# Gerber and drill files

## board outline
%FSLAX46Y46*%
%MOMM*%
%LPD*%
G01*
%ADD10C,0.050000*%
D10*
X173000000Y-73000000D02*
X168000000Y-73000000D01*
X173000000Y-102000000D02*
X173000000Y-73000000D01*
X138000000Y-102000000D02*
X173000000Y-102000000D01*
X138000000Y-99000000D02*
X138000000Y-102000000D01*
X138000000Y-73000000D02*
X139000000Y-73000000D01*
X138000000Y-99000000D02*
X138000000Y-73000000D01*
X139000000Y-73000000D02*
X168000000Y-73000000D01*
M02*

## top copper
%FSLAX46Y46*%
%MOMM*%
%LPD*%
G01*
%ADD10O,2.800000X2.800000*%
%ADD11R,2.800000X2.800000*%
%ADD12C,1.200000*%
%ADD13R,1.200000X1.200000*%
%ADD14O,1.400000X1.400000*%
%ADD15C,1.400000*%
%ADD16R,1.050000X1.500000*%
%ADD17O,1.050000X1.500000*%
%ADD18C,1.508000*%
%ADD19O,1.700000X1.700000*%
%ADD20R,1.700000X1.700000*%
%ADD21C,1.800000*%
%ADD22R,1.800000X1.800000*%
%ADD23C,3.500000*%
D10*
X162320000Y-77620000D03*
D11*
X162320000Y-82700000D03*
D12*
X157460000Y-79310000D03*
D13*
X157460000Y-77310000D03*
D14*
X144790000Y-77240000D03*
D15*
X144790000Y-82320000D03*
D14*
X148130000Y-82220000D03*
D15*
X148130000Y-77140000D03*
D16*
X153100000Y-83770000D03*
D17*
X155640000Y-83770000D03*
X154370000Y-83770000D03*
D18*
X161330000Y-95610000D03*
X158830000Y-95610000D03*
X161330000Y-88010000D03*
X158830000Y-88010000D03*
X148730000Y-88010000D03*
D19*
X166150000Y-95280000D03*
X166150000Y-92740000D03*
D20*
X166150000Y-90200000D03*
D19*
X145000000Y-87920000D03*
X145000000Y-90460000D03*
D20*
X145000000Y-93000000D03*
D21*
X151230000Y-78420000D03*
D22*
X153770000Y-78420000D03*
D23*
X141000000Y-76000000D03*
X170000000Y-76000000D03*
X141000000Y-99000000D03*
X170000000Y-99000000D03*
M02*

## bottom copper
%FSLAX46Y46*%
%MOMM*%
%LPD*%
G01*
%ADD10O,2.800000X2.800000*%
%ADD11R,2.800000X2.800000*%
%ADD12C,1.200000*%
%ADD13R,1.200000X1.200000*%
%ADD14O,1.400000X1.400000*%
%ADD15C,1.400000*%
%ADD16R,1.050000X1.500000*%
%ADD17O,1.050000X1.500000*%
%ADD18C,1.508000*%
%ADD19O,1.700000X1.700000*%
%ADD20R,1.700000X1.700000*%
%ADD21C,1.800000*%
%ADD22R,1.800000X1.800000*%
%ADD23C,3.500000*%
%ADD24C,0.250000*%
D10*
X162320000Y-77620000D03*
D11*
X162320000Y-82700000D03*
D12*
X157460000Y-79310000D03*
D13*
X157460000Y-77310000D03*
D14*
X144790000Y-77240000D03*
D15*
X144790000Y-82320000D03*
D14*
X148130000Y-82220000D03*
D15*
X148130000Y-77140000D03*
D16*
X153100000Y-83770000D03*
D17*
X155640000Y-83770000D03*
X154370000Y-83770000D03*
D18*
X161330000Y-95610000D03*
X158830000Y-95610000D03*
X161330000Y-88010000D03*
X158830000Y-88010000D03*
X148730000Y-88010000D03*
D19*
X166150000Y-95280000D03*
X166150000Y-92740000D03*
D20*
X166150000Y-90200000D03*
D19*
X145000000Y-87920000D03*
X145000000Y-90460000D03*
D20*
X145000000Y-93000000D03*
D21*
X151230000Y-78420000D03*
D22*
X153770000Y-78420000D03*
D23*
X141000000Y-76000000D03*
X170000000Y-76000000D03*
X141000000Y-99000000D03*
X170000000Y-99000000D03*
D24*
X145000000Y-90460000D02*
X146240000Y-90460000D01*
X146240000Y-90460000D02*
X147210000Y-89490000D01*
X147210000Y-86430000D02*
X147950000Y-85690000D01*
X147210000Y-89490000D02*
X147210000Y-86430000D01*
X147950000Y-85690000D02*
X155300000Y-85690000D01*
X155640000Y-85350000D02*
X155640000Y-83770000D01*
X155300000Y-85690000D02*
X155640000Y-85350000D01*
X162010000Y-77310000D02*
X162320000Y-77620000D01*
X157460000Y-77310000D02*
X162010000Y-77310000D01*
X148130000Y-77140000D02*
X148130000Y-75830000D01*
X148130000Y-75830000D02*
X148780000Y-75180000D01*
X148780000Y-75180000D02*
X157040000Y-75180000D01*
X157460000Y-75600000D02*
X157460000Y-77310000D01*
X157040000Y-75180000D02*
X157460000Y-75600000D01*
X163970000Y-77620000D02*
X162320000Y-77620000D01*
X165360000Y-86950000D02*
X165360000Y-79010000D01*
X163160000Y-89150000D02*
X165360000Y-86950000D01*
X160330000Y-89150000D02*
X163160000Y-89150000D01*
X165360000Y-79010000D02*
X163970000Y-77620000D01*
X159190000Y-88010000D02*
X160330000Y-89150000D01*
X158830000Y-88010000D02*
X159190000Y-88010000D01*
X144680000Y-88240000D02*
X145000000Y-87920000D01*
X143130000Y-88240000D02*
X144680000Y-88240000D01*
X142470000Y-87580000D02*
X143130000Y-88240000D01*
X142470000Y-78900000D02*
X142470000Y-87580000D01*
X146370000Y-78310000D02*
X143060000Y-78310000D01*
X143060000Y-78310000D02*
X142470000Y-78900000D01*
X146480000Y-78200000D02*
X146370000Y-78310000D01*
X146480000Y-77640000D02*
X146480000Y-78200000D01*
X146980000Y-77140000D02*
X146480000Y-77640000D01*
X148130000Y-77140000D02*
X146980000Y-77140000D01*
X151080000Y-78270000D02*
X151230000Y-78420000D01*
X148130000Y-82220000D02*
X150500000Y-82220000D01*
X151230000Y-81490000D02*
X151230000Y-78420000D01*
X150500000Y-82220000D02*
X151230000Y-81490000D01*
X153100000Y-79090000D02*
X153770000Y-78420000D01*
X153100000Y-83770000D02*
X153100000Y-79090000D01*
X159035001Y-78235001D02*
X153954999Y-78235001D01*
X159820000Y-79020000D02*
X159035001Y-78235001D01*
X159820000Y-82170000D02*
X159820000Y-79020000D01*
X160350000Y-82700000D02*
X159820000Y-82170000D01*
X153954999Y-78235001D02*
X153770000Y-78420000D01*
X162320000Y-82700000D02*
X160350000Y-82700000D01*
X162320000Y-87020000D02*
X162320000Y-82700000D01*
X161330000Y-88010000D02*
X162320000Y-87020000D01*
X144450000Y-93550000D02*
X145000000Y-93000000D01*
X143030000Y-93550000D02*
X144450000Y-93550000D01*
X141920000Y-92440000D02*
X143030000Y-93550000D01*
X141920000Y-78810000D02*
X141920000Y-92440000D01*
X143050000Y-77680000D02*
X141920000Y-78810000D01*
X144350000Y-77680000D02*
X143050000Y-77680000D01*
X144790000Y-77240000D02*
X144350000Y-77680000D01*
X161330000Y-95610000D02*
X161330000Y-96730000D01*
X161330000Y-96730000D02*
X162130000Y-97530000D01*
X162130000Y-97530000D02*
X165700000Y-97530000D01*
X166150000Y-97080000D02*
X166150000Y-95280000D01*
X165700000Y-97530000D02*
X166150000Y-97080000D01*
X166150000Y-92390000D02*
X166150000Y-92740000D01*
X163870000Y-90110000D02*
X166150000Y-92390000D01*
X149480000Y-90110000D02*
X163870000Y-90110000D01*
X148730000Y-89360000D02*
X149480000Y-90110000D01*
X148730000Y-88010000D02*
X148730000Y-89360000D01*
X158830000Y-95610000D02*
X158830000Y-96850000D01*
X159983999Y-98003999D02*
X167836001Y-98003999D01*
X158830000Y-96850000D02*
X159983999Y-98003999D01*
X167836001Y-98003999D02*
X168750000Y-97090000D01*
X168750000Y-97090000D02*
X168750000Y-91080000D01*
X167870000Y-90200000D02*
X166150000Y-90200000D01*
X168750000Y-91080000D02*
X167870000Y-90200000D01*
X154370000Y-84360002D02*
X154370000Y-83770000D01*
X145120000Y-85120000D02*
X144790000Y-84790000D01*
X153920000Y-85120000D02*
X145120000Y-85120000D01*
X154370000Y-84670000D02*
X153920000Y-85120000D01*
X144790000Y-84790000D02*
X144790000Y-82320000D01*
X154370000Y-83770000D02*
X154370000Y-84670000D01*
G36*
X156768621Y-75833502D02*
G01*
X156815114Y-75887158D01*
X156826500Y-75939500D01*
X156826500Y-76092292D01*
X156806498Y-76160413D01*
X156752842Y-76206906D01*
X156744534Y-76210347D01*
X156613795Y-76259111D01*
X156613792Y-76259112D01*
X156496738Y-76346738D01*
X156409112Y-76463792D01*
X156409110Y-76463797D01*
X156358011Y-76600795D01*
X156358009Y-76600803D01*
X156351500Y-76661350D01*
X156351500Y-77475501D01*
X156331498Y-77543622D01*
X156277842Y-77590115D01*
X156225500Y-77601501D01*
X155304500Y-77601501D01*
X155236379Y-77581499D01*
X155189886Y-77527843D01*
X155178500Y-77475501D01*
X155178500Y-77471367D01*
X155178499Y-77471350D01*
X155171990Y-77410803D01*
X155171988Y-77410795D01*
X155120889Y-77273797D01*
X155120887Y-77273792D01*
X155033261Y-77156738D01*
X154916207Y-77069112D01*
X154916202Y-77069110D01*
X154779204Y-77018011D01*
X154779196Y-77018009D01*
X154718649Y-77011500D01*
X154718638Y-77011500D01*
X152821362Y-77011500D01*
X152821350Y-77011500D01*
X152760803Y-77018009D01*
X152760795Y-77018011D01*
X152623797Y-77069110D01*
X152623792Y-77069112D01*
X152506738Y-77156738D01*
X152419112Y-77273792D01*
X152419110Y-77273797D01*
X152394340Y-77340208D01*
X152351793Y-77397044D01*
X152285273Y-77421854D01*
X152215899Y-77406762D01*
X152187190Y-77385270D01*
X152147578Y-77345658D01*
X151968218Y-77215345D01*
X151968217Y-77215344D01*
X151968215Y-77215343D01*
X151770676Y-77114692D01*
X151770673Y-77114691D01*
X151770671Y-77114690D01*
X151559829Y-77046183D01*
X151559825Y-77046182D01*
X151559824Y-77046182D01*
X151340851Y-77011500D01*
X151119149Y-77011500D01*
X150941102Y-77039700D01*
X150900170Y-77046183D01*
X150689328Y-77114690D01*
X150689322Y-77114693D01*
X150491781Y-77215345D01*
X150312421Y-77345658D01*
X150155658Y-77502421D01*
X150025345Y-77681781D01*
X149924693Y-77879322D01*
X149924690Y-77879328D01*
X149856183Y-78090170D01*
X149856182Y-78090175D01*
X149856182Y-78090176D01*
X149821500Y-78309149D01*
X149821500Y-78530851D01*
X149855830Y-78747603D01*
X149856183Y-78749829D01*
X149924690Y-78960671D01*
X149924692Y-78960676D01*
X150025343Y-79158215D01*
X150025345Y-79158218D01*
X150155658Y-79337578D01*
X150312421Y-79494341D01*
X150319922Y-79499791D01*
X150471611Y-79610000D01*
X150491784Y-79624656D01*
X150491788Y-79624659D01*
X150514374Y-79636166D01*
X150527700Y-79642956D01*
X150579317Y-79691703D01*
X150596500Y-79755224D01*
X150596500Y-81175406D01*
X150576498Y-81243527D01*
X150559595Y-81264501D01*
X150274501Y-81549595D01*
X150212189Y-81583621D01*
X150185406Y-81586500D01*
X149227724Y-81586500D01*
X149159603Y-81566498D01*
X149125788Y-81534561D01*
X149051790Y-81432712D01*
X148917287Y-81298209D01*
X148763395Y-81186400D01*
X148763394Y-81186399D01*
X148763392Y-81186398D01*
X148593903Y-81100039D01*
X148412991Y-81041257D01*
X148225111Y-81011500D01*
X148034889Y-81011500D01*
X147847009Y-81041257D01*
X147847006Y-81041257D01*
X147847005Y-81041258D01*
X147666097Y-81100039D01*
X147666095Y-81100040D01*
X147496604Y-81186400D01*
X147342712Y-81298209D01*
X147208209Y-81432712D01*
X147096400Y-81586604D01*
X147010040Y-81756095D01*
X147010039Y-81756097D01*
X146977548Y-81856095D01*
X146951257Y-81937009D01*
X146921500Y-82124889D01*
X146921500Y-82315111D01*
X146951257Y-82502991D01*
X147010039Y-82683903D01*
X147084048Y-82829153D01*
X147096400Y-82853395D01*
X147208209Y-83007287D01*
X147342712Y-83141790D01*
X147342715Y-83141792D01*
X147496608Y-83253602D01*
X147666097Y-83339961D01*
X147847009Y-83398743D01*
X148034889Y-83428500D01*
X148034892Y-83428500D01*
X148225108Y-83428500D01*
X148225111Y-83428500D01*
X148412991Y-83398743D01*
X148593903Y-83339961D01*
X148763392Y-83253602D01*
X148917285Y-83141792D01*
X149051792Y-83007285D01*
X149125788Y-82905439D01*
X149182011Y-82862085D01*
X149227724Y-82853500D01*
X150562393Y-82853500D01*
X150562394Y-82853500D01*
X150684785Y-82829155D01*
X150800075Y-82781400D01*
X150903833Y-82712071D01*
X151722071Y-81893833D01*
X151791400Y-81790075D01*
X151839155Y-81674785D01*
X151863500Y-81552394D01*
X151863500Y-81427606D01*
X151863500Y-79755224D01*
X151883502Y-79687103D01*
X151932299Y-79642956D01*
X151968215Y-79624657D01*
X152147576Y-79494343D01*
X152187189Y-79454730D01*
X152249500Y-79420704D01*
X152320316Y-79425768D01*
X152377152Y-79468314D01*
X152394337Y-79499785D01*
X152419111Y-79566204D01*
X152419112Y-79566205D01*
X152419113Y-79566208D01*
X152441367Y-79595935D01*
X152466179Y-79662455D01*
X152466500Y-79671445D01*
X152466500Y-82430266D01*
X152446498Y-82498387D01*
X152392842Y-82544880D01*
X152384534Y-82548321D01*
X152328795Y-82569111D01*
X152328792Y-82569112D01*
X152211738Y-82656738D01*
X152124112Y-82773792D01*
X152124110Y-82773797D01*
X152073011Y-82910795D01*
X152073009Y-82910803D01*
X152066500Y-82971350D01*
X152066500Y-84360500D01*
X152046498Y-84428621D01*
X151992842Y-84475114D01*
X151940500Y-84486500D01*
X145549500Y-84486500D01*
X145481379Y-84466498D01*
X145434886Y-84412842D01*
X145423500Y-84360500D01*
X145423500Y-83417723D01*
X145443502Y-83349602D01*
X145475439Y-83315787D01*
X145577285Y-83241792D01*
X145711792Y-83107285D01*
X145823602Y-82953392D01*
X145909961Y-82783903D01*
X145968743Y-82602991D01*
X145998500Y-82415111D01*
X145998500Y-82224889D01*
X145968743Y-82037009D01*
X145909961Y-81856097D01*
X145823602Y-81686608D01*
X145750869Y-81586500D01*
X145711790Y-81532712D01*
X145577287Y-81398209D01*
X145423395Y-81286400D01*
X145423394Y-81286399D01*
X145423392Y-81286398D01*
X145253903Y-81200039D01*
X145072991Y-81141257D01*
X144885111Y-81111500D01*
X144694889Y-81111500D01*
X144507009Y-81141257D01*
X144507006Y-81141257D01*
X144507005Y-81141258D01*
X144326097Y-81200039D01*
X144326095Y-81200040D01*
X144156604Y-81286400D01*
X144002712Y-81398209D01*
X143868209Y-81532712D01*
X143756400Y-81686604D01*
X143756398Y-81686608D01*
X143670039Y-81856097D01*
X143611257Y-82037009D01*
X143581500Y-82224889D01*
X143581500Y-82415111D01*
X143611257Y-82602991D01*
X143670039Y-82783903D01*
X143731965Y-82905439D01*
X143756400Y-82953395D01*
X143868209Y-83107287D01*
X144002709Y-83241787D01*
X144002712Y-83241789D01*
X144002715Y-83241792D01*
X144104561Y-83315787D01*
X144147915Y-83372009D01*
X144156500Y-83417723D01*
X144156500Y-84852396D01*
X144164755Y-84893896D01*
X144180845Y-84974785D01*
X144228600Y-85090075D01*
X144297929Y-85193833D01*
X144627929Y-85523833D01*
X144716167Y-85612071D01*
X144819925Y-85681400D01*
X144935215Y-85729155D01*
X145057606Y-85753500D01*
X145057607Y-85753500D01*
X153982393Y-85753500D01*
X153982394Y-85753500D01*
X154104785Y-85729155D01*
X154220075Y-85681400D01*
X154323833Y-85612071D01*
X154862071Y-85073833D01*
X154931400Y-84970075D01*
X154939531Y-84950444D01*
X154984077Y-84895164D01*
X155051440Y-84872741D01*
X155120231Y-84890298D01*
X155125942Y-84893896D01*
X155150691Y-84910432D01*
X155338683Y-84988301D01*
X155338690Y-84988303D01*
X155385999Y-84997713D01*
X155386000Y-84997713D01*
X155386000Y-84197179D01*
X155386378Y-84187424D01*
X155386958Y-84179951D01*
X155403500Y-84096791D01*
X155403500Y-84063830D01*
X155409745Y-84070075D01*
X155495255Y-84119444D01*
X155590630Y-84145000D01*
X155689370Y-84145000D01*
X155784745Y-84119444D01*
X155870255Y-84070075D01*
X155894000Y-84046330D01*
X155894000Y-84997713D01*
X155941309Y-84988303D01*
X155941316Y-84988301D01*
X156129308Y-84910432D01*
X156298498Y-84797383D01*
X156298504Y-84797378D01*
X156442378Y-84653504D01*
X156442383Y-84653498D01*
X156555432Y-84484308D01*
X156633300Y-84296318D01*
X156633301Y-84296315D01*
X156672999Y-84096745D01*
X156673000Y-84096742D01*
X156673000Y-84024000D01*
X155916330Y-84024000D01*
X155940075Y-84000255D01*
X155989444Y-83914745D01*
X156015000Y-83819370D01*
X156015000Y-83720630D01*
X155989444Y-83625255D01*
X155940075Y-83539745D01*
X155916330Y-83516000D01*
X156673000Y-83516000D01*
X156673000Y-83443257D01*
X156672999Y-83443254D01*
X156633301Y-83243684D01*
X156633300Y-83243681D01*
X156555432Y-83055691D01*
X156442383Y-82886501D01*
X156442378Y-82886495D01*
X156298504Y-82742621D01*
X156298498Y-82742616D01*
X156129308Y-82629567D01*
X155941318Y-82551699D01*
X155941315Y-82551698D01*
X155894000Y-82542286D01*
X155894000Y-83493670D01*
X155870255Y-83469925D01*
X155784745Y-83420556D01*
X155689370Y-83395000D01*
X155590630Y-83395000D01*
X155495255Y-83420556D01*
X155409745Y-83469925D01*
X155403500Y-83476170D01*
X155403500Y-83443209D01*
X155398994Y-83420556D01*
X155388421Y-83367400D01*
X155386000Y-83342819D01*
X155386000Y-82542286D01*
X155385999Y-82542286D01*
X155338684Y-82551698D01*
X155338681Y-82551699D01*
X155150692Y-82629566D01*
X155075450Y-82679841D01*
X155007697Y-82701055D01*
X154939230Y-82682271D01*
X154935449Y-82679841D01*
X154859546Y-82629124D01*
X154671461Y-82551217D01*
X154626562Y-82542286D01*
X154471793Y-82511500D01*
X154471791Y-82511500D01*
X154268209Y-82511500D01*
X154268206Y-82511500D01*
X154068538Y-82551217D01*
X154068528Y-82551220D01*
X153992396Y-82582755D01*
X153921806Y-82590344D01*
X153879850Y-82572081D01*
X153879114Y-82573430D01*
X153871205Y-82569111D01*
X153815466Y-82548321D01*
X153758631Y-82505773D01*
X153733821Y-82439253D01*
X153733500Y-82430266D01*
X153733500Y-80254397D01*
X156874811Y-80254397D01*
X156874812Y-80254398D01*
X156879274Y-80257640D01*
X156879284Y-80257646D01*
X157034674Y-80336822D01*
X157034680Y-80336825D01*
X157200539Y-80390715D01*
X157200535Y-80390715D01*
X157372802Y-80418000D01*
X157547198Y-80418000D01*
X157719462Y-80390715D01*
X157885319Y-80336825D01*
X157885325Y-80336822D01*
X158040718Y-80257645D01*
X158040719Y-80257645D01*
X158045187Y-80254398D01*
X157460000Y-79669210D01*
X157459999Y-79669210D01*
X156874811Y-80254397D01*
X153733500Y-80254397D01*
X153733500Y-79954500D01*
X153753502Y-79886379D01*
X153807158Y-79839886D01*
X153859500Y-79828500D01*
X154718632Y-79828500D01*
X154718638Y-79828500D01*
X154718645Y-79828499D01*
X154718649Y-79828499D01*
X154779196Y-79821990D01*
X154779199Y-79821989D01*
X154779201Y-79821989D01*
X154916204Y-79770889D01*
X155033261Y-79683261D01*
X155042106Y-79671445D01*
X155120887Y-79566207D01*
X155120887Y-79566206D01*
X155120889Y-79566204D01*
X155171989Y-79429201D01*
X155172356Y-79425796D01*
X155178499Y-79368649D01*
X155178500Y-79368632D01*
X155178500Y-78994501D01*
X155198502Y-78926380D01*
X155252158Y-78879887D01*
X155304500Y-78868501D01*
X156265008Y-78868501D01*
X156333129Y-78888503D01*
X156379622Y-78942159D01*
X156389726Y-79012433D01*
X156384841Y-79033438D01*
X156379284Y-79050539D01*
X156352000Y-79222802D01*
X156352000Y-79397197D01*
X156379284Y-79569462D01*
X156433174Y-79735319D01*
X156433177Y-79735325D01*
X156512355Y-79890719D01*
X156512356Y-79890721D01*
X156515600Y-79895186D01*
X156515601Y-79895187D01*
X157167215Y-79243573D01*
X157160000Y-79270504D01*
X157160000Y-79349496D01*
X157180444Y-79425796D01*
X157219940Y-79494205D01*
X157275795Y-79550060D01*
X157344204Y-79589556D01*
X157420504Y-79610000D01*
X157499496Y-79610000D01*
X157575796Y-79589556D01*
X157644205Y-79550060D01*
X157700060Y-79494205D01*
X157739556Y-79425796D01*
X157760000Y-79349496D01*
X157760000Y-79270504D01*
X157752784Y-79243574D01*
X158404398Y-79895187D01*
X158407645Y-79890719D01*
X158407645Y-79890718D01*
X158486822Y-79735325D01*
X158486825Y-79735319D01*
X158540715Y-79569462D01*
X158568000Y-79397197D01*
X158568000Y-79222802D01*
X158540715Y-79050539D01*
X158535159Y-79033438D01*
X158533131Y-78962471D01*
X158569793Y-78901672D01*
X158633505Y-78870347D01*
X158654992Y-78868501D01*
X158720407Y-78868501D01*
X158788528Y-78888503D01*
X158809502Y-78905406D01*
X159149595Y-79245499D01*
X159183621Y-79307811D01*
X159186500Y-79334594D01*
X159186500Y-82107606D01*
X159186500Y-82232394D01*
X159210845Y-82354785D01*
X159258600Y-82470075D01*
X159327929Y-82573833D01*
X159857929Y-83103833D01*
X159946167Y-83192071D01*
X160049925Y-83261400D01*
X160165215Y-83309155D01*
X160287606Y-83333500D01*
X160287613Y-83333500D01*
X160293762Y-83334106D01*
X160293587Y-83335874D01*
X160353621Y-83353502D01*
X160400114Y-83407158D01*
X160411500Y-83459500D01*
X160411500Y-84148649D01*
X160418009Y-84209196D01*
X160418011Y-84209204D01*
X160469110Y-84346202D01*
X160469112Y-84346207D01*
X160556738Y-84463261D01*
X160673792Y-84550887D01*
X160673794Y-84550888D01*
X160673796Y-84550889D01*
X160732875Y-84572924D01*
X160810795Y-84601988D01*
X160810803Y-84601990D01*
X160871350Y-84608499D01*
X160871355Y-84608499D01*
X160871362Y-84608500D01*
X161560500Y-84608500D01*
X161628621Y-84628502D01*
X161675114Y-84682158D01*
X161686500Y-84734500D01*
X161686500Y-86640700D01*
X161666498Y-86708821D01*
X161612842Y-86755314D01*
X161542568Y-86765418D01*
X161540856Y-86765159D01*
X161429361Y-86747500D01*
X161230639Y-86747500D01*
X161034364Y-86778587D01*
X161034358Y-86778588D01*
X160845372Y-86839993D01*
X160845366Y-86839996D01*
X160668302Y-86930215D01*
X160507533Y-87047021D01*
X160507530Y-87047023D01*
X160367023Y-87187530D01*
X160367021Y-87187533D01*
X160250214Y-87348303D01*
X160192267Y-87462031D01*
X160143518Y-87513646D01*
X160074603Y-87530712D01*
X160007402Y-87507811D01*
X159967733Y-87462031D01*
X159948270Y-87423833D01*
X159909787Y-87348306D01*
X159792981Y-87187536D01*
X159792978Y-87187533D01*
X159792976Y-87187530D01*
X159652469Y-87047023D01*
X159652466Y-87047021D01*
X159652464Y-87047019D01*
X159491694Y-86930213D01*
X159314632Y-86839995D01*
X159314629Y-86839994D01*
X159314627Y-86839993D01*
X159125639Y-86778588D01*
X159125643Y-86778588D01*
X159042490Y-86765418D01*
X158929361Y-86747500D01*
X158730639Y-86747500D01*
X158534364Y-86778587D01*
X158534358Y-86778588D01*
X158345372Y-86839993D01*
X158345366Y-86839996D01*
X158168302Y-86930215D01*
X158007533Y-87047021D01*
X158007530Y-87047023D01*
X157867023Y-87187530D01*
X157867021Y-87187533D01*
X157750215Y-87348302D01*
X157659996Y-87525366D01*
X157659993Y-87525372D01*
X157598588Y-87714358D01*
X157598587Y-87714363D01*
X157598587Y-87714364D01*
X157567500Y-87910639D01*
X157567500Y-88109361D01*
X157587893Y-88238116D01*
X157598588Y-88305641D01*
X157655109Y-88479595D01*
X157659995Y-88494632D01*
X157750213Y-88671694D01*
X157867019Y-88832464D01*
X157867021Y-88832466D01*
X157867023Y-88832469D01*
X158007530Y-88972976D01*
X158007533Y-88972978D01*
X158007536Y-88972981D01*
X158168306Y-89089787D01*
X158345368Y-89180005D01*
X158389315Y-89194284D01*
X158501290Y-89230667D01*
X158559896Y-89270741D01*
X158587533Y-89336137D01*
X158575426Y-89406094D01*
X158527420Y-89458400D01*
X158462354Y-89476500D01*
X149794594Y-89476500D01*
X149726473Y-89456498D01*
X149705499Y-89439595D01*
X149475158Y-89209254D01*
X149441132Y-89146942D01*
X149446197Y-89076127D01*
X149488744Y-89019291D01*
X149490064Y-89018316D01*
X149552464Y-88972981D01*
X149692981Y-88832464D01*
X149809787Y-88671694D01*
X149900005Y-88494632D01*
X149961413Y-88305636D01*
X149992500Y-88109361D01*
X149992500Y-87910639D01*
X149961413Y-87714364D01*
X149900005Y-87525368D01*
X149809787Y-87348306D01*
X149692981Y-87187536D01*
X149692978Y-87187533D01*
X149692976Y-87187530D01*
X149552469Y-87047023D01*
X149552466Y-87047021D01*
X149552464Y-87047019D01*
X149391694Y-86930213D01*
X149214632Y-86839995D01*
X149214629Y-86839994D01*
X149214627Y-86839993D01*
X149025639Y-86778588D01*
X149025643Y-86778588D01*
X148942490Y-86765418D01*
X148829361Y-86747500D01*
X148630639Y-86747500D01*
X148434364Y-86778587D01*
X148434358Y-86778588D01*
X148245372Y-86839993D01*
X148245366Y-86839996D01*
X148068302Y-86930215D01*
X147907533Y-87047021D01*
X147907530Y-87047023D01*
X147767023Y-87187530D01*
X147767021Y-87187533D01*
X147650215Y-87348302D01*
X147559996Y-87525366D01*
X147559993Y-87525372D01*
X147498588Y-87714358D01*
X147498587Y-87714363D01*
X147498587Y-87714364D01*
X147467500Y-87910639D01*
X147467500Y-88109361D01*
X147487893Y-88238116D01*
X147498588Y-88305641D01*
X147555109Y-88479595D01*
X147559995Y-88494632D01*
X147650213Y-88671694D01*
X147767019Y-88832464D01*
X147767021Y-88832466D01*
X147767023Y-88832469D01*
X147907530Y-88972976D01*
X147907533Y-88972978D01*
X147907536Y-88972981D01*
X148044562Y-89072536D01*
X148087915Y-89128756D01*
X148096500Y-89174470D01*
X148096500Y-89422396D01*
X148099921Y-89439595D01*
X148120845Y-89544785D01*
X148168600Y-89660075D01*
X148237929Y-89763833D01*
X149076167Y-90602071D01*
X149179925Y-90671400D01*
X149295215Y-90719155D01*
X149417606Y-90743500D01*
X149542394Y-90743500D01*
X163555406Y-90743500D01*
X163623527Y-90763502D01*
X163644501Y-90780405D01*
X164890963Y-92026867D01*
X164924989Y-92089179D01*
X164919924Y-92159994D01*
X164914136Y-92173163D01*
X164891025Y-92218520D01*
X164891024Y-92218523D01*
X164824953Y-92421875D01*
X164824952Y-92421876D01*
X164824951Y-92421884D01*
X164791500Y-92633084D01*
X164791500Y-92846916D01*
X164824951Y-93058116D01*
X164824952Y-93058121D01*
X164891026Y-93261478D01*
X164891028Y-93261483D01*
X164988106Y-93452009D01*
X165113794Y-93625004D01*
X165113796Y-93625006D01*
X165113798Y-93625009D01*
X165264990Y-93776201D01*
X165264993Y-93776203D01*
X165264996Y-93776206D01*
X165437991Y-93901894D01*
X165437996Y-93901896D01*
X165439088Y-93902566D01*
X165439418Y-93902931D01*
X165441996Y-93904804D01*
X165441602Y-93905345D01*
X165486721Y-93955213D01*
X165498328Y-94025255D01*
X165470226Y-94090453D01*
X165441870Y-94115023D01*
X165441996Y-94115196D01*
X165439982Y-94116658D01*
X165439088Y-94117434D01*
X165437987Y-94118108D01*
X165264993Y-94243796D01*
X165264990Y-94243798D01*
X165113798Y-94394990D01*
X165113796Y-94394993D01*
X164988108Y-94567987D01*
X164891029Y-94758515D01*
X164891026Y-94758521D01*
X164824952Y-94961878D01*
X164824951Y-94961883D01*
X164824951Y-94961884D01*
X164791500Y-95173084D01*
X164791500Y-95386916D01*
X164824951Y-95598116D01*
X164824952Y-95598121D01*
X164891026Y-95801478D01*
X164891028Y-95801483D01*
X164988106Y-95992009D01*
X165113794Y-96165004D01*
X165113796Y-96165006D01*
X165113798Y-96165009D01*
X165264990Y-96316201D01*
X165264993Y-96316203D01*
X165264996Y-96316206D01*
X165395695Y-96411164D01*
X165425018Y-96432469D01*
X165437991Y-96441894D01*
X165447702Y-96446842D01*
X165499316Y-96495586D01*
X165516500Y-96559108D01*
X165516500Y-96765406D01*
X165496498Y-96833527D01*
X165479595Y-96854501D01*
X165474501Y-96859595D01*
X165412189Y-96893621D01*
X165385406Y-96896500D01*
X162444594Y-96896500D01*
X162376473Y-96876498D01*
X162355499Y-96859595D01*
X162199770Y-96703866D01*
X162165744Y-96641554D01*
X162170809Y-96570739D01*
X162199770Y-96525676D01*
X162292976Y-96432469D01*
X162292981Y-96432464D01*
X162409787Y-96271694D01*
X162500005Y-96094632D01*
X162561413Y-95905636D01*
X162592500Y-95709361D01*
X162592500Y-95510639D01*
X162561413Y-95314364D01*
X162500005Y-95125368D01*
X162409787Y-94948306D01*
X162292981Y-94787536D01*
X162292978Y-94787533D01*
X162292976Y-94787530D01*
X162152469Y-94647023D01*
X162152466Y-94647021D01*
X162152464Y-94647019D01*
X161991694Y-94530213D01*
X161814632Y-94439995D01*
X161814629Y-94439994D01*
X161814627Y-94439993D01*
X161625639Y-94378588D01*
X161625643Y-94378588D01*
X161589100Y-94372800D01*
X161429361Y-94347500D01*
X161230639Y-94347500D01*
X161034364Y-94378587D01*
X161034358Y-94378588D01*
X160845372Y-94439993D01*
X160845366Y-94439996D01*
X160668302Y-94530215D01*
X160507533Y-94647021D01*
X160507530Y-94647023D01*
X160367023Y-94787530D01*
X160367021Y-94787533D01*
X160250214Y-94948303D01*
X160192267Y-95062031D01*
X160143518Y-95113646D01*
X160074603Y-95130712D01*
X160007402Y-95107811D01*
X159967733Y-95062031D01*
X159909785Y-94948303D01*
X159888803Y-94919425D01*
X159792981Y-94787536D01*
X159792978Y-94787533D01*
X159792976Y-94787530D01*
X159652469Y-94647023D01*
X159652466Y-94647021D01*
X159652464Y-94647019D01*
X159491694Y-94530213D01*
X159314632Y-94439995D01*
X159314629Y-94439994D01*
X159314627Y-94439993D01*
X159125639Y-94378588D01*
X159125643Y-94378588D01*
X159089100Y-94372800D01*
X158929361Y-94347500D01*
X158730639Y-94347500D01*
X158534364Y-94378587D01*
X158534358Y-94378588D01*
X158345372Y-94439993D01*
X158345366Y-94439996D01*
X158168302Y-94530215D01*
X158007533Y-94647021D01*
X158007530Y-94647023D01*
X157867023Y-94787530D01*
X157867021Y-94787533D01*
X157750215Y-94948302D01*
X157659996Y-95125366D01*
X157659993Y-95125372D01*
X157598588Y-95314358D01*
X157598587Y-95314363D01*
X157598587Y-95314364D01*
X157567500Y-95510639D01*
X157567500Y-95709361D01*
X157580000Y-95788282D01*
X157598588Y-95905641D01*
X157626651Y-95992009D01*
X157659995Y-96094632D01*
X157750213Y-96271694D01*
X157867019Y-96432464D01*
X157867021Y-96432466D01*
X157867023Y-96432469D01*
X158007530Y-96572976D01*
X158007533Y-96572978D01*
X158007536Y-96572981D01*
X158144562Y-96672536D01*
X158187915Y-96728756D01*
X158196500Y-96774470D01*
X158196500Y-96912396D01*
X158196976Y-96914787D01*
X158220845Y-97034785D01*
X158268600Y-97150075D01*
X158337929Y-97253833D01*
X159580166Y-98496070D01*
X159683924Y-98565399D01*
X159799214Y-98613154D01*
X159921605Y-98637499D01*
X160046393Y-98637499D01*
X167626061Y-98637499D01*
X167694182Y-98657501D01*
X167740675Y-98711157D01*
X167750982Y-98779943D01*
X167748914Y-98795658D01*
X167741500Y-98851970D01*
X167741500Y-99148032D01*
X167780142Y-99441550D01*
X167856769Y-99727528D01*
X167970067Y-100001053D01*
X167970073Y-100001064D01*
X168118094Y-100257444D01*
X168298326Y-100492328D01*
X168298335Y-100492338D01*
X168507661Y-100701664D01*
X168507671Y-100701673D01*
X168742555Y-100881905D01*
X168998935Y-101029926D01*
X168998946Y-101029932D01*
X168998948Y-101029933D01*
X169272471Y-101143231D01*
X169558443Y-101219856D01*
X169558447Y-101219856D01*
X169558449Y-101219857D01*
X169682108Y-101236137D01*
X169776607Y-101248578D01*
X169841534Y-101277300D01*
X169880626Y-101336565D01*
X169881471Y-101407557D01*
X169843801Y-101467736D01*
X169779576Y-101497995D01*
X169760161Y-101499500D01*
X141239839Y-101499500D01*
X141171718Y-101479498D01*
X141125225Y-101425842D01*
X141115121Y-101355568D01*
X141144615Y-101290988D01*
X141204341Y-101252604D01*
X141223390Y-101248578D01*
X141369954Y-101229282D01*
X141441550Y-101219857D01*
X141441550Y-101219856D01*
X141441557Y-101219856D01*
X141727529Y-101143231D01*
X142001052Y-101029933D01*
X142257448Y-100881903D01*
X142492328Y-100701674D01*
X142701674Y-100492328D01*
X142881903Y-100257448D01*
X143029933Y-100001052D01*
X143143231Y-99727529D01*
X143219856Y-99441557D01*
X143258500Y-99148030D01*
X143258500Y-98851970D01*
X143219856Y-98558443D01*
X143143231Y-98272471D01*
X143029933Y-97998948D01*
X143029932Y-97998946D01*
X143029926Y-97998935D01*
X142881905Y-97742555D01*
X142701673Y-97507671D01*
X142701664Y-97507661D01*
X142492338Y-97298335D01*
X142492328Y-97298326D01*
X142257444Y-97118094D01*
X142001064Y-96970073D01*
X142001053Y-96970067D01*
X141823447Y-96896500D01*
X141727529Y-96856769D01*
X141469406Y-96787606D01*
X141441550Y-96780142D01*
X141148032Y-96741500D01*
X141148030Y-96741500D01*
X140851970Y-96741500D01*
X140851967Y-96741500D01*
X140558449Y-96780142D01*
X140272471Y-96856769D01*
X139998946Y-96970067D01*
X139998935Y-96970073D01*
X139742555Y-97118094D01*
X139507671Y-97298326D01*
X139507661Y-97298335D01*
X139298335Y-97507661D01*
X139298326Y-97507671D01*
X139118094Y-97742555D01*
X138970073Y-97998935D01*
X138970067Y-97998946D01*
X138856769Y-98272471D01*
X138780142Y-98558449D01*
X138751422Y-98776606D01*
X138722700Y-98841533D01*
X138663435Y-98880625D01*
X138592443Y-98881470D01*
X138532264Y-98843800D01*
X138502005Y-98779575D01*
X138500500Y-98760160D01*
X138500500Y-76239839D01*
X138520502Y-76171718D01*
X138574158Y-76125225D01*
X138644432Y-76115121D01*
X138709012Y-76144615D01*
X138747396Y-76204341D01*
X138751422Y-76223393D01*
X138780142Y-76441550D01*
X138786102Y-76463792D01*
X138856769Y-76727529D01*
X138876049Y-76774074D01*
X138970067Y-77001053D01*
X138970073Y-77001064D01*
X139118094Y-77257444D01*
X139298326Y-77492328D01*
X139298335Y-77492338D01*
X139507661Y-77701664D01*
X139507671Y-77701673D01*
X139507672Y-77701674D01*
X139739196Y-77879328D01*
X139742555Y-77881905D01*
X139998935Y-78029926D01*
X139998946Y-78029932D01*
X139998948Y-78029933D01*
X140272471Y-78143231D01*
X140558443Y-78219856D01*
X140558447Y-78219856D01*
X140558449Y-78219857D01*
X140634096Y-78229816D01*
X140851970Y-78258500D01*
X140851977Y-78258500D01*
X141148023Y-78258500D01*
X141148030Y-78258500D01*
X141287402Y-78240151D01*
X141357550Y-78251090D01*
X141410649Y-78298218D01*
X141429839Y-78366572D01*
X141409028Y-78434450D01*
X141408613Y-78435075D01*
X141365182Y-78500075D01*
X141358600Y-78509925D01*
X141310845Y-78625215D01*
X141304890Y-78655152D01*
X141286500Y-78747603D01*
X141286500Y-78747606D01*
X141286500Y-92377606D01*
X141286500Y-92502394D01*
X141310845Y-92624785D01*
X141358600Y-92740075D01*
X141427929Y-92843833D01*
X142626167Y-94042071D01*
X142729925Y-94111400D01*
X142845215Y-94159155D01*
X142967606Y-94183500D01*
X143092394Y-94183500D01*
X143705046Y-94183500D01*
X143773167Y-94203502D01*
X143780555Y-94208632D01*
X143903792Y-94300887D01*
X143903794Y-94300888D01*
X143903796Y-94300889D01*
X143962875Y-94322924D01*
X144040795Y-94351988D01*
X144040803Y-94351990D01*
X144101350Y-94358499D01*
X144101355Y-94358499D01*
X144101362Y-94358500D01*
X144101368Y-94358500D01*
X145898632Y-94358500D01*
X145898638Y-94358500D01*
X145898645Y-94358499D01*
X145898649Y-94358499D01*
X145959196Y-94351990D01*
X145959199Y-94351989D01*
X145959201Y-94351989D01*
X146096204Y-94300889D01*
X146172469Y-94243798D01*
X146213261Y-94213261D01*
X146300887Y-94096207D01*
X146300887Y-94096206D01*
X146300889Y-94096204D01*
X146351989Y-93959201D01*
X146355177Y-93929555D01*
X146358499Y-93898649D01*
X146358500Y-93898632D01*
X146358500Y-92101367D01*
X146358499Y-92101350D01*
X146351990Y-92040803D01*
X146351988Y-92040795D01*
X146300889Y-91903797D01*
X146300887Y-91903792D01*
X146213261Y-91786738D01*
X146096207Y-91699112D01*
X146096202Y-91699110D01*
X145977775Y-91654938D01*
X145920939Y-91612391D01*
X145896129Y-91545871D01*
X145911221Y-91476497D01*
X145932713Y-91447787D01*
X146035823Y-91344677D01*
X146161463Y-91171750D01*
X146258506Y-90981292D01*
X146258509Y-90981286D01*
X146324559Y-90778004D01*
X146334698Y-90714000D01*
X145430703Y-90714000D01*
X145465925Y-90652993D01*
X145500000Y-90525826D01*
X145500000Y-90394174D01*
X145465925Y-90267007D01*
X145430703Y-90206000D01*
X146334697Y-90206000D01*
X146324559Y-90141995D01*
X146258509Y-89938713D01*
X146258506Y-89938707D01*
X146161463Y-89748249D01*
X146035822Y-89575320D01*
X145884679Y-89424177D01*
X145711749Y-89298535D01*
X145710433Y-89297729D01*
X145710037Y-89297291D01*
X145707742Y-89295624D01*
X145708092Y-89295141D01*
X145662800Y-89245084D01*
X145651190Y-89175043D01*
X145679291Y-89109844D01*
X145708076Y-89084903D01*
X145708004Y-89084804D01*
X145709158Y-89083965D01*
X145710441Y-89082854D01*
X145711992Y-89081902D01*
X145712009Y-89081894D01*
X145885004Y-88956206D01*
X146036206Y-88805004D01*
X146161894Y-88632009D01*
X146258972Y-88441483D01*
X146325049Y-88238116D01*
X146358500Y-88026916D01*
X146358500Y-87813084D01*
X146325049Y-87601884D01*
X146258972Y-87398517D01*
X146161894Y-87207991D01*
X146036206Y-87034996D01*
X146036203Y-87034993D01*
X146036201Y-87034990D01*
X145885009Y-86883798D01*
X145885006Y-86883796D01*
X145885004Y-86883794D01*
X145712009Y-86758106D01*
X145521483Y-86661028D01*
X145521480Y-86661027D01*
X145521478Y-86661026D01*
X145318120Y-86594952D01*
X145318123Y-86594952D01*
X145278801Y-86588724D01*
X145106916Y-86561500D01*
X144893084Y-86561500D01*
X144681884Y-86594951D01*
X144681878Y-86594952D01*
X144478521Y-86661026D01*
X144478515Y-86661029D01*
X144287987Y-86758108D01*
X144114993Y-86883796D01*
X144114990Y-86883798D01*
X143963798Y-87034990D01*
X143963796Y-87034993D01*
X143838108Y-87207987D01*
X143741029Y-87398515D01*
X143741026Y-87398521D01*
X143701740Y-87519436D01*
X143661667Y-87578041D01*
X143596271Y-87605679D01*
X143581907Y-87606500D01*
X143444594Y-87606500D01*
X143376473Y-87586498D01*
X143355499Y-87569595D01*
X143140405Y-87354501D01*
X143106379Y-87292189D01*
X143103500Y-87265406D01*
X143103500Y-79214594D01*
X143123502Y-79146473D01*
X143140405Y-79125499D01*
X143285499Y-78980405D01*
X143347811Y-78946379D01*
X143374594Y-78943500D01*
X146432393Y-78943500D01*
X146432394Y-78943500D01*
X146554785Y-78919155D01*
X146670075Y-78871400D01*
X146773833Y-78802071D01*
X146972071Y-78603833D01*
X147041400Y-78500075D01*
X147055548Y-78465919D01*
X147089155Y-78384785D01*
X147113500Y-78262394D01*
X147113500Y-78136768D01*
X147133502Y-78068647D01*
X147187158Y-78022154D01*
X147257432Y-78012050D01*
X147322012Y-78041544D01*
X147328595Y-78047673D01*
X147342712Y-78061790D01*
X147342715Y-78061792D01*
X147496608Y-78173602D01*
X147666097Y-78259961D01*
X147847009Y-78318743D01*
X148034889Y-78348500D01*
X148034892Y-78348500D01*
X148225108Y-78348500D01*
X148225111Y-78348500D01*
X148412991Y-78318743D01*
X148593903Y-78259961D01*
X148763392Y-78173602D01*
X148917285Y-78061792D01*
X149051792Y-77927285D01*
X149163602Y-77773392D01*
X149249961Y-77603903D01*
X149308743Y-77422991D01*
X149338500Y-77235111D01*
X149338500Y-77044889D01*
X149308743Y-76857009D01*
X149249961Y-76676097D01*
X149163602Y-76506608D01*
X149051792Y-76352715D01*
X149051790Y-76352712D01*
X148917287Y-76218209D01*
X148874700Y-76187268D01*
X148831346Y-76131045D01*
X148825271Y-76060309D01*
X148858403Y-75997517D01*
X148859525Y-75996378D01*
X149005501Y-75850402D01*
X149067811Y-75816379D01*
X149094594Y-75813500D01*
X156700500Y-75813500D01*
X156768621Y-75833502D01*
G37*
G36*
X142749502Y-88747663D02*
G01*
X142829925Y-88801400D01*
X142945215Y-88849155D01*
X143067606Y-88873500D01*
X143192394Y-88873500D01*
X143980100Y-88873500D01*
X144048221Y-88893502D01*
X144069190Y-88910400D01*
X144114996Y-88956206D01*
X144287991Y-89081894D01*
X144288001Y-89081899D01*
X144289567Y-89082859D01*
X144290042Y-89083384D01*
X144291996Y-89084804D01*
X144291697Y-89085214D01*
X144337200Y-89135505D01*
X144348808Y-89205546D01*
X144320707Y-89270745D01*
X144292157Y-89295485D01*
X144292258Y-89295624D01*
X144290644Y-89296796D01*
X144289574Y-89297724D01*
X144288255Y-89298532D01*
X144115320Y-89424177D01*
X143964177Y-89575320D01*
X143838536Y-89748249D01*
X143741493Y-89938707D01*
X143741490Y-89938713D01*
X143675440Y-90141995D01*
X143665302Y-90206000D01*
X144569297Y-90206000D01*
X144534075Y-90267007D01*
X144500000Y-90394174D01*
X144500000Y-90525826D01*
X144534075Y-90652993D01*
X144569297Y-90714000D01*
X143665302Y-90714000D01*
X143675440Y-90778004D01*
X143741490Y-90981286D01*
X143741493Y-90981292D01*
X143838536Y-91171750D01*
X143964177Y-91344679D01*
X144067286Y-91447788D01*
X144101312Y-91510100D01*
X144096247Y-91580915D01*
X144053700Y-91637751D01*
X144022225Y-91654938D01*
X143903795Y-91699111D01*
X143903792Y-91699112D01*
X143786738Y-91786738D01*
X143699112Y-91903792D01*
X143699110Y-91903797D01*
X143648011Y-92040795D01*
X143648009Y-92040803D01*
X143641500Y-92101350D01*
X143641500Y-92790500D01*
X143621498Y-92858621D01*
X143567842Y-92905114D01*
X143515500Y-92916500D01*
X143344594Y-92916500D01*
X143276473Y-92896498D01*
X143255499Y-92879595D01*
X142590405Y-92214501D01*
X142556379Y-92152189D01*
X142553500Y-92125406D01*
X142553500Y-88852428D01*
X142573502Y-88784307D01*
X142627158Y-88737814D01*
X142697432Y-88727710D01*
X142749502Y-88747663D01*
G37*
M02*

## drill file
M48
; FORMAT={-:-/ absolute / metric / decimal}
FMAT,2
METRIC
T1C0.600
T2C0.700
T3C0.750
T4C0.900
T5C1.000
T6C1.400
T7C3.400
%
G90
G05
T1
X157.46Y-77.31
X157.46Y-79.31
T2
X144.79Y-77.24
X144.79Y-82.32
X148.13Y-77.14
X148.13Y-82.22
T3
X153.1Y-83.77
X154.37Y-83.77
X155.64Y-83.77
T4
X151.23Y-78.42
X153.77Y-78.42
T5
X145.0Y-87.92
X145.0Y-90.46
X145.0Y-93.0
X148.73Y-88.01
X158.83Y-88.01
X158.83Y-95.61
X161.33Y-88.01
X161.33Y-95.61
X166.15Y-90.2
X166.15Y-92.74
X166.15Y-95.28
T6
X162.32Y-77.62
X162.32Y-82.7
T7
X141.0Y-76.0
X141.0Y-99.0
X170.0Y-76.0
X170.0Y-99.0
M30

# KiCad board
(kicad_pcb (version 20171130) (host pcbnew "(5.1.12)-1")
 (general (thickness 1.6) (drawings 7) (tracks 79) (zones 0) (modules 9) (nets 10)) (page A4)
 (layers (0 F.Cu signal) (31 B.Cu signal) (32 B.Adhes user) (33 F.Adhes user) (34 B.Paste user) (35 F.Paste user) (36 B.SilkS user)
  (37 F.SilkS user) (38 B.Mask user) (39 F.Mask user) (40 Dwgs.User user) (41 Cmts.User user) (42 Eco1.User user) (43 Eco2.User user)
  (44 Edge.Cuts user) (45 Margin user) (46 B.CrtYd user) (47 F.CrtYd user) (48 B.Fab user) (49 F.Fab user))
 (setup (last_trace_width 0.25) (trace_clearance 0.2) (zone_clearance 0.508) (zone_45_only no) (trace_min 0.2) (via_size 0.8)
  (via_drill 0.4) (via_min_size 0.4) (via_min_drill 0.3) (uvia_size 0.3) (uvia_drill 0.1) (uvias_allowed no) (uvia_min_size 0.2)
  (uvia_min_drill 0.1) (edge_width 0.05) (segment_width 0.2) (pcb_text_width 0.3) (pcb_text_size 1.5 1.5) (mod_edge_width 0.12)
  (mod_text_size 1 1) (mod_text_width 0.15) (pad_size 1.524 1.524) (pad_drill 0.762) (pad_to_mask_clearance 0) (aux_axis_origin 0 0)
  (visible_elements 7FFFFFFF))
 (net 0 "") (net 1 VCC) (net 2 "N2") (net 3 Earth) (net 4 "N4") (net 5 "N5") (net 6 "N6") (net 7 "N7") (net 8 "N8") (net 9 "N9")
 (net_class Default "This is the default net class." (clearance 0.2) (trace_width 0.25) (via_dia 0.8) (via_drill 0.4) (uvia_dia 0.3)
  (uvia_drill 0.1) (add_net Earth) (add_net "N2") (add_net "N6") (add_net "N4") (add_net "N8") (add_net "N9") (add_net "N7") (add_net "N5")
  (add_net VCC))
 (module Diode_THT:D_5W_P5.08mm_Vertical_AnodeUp (layer F.Cu) (at 162.32 82.7 90)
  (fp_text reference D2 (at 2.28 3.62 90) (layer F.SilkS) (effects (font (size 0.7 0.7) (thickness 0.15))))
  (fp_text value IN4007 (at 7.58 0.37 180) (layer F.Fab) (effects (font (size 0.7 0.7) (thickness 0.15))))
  (pad 2 thru_hole oval (at 5.08 0 90) (size 2.8 2.8) (drill 1.4) (layers *.Cu *.Mask) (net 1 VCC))
  (pad 1 thru_hole rect (at 0 0 90) (size 2.8 2.8) (drill 1.4) (layers *.Cu *.Mask) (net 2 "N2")))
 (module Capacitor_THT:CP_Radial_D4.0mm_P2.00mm (layer F.Cu) (at 157.46 77.31 270)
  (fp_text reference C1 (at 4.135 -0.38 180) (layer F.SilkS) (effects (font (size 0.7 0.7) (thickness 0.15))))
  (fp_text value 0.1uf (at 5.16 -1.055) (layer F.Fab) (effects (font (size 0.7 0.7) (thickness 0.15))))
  (pad 2 thru_hole circle (at 2 0 270) (size 1.2 1.2) (drill 0.6) (layers *.Cu *.Mask) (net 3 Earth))
  (pad 1 thru_hole rect (at 0 0 270) (size 1.2 1.2) (drill 0.6) (layers *.Cu *.Mask) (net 1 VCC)))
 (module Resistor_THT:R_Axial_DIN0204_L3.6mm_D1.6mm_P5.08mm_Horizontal (layer F.Cu) (at 144.79 82.32 90)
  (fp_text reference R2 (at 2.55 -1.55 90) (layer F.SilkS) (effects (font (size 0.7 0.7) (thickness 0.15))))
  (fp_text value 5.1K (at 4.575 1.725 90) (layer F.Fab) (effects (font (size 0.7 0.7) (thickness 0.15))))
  (pad 2 thru_hole oval (at 5.08 0 90) (size 1.4 1.4) (drill 0.7) (layers *.Cu *.Mask) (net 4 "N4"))
  (pad 1 thru_hole circle (at 0 0 90) (size 1.4 1.4) (drill 0.7) (layers *.Cu *.Mask) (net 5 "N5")))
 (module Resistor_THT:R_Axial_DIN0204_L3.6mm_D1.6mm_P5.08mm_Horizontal (layer F.Cu) (at 148.13 77.14 270)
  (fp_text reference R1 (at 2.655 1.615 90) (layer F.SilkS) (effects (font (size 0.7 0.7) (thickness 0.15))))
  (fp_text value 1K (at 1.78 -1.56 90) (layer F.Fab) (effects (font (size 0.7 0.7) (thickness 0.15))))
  (pad 2 thru_hole oval (at 5.08 0 270) (size 1.4 1.4) (drill 0.7) (layers *.Cu *.Mask) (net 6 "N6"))
  (pad 1 thru_hole circle (at 0 0 270) (size 1.4 1.4) (drill 0.7) (layers *.Cu *.Mask) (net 1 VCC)))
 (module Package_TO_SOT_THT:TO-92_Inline (layer F.Cu) (at 153.1 83.77)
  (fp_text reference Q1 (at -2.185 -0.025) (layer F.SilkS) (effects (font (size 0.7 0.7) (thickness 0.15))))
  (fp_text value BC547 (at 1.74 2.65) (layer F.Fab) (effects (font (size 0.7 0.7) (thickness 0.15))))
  (pad 1 thru_hole rect (at 0 0) (size 1.05 1.5) (drill 0.75) (layers *.Cu *.Mask) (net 2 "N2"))
  (pad 3 thru_hole oval (at 2.54 0) (size 1.05 1.5) (drill 0.75) (layers *.Cu *.Mask) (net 3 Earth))
  (pad 2 thru_hole oval (at 1.27 0) (size 1.05 1.5) (drill 0.75) (layers *.Cu *.Mask) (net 5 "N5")))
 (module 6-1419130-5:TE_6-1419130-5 (layer F.Cu) (at 155.03 91.81 180)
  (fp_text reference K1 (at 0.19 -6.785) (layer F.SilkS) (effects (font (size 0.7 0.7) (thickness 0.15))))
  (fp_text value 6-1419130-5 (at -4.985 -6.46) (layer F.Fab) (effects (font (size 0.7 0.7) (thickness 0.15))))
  (pad 12 thru_hole circle (at -6.3 -3.8 180) (size 1.508 1.508) (drill 1) (layers *.Cu *.Mask) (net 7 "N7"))
  (pad 14 thru_hole circle (at -3.8 -3.8 180) (size 1.508 1.508) (drill 1) (layers *.Cu *.Mask) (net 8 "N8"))
  (pad A1 thru_hole circle (at -6.3 3.8 180) (size 1.508 1.508) (drill 1) (layers *.Cu *.Mask) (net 2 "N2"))
  (pad A2 thru_hole circle (at -3.8 3.8 180) (size 1.508 1.508) (drill 1) (layers *.Cu *.Mask) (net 1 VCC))
  (pad 11 thru_hole circle (at 6.3 3.8 180) (size 1.508 1.508) (drill 1) (layers *.Cu *.Mask) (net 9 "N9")))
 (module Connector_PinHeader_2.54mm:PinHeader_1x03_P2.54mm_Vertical (layer F.Cu) (at 166.15 90.2)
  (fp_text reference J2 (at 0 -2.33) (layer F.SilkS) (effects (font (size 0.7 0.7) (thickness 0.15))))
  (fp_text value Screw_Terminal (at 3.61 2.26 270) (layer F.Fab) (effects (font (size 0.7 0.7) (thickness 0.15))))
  (pad 3 thru_hole oval (at 0 5.08) (size 1.7 1.7) (drill 1) (layers *.Cu *.Mask) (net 7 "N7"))
  (pad 2 thru_hole oval (at 0 2.54) (size 1.7 1.7) (drill 1) (layers *.Cu *.Mask) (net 9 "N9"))
  (pad 1 thru_hole rect (at 0 0) (size 1.7 1.7) (drill 1) (layers *.Cu *.Mask) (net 8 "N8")))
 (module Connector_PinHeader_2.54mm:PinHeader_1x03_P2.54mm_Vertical (layer F.Cu) (at 145 93 180)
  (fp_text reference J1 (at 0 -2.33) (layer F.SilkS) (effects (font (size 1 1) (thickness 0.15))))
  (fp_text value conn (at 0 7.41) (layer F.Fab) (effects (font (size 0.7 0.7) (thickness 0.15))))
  (pad 3 thru_hole oval (at 0 5.08 180) (size 1.7 1.7) (drill 1) (layers *.Cu *.Mask) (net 1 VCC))
  (pad 2 thru_hole oval (at 0 2.54 180) (size 1.7 1.7) (drill 1) (layers *.Cu *.Mask) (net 3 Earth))
  (pad 1 thru_hole rect (at 0 0 180) (size 1.7 1.7) (drill 1) (layers *.Cu *.Mask) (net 4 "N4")))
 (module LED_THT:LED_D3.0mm (layer F.Cu) (at 153.77 78.42 180)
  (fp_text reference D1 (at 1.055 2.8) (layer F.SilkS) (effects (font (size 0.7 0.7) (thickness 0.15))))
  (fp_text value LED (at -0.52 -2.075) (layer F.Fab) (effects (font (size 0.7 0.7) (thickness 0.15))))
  (pad 2 thru_hole circle (at 2.54 0 180) (size 1.8 1.8) (drill 0.9) (layers *.Cu *.Mask) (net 6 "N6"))
  (pad 1 thru_hole rect (at 0 0 180) (size 1.8 1.8) (drill 0.9) (layers *.Cu *.Mask) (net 2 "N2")))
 (gr_line (start 173 73) (end 168 73) (layer Edge.Cuts) (width 0.05))
 (gr_line (start 173 102) (end 173 73) (layer Edge.Cuts) (width 0.05))
 (gr_line (start 138 102) (end 173 102) (layer Edge.Cuts) (width 0.05))
 (gr_line (start 138 99) (end 138 102) (layer Edge.Cuts) (width 0.05))
 (gr_line (start 138 73) (end 139 73) (layer Edge.Cuts) (width 0.05))
 (gr_line (start 138 99) (end 138 73) (layer Edge.Cuts) (width 0.05))
 (gr_line (start 139 73) (end 168 73) (layer Edge.Cuts) (width 0.05))
 (via (at 141 76) (size 3.5) (drill 3.4) (layers F.Cu B.Cu) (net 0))
 (via (at 170 76) (size 3.5) (drill 3.4) (layers F.Cu B.Cu) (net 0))
 (via (at 141 99) (size 3.5) (drill 3.4) (layers F.Cu B.Cu) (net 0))
 (via (at 170 99) (size 3.5) (drill 3.4) (layers F.Cu B.Cu) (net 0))
 (segment (start 145 90.46) (end 146.24 90.46) (width 0.25) (layer B.Cu) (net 3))
 (segment (start 146.24 90.46) (end 147.21 89.49) (width 0.25) (layer B.Cu) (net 3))
 (segment (start 147.21 86.43) (end 147.95 85.69) (width 0.25) (layer B.Cu) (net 3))
 (segment (start 147.21 89.49) (end 147.21 86.43) (width 0.25) (layer B.Cu) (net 3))
 (segment (start 147.95 85.69) (end 155.3 85.69) (width 0.25) (layer B.Cu) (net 3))
 (segment (start 155.64 85.35) (end 155.64 83.77) (width 0.25) (layer B.Cu) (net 3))
 (segment (start 155.3 85.69) (end 155.64 85.35) (width 0.25) (layer B.Cu) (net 3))
 (segment (start 162.01 77.31) (end 162.32 77.62) (width 0.25) (layer B.Cu) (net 1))
 (segment (start 157.46 77.31) (end 162.01 77.31) (width 0.25) (layer B.Cu) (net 1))
 (segment (start 148.13 77.14) (end 148.13 75.83) (width 0.25) (layer B.Cu) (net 1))
 (segment (start 148.13 75.83) (end 148.78 75.18) (width 0.25) (layer B.Cu) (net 1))
 (segment (start 148.78 75.18) (end 157.04 75.18) (width 0.25) (layer B.Cu) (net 1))
 (segment (start 157.46 75.6) (end 157.46 77.31) (width 0.25) (layer B.Cu) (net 1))
 (segment (start 157.04 75.18) (end 157.46 75.6) (width 0.25) (layer B.Cu) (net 1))
 (segment (start 163.97 77.62) (end 162.32 77.62) (width 0.25) (layer B.Cu) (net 1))
 (segment (start 165.36 86.95) (end 165.36 79.01) (width 0.25) (layer B.Cu) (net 1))
 (segment (start 163.16 89.15) (end 165.36 86.95) (width 0.25) (layer B.Cu) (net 1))
 (segment (start 160.33 89.15) (end 163.16 89.15) (width 0.25) (layer B.Cu) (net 1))
 (segment (start 165.36 79.01) (end 163.97 77.62) (width 0.25) (layer B.Cu) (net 1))
 (segment (start 159.19 88.01) (end 160.33 89.15) (width 0.25) (layer B.Cu) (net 1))
 (segment (start 158.83 88.01) (end 159.19 88.01) (width 0.25) (layer B.Cu) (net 1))
 (segment (start 144.68 88.24) (end 145 87.92) (width 0.25) (layer B.Cu) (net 1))
 (segment (start 143.13 88.24) (end 144.68 88.24) (width 0.25) (layer B.Cu) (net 1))
 (segment (start 142.47 87.58) (end 143.13 88.24) (width 0.25) (layer B.Cu) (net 1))
 (segment (start 142.47 78.9) (end 142.47 87.58) (width 0.25) (layer B.Cu) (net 1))
 (segment (start 146.37 78.31) (end 143.06 78.31) (width 0.25) (layer B.Cu) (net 1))
 (segment (start 143.06 78.31) (end 142.47 78.9) (width 0.25) (layer B.Cu) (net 1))
 (segment (start 146.48 78.2) (end 146.37 78.31) (width 0.25) (layer B.Cu) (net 1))
 (segment (start 146.48 77.64) (end 146.48 78.2) (width 0.25) (layer B.Cu) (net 1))
 (segment (start 146.98 77.14) (end 146.48 77.64) (width 0.25) (layer B.Cu) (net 1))
 (segment (start 148.13 77.14) (end 146.98 77.14) (width 0.25) (layer B.Cu) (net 1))
 (segment (start 151.08 78.27) (end 151.23 78.42) (width 0.25) (layer B.Cu) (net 6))
 (segment (start 148.13 82.22) (end 150.5 82.22) (width 0.25) (layer B.Cu) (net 6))
 (segment (start 151.23 81.49) (end 151.23 78.42) (width 0.25) (layer B.Cu) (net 6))
 (segment (start 150.5 82.22) (end 151.23 81.49) (width 0.25) (layer B.Cu) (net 6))
 (segment (start 153.1 79.09) (end 153.77 78.42) (width 0.25) (layer B.Cu) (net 2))
 (segment (start 153.1 83.77) (end 153.1 79.09) (width 0.25) (layer B.Cu) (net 2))
 (segment (start 159.035001 78.235001) (end 153.954999 78.235001) (width 0.25) (layer B.Cu) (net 2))
 (segment (start 159.82 79.02) (end 159.035001 78.235001) (width 0.25) (layer B.Cu) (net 2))
 (segment (start 159.82 82.17) (end 159.82 79.02) (width 0.25) (layer B.Cu) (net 2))
 (segment (start 160.35 82.7) (end 159.82 82.17) (width 0.25) (layer B.Cu) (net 2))
 (segment (start 153.954999 78.235001) (end 153.77 78.42) (width 0.25) (layer B.Cu) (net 2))
 (segment (start 162.32 82.7) (end 160.35 82.7) (width 0.25) (layer B.Cu) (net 2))
 (segment (start 162.32 87.02) (end 162.32 82.7) (width 0.25) (layer B.Cu) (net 2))
 (segment (start 161.33 88.01) (end 162.32 87.02) (width 0.25) (layer B.Cu) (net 2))
 (segment (start 144.45 93.55) (end 145 93) (width 0.25) (layer B.Cu) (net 4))
 (segment (start 143.03 93.55) (end 144.45 93.55) (width 0.25) (layer B.Cu) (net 4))
 (segment (start 141.92 92.44) (end 143.03 93.55) (width 0.25) (layer B.Cu) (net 4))
 (segment (start 141.92 78.81) (end 141.92 92.44) (width 0.25) (layer B.Cu) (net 4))
 (segment (start 143.05 77.68) (end 141.92 78.81) (width 0.25) (layer B.Cu) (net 4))
 (segment (start 144.35 77.68) (end 143.05 77.68) (width 0.25) (layer B.Cu) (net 4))
 (segment (start 144.79 77.24) (end 144.35 77.68) (width 0.25) (layer B.Cu) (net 4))
 (segment (start 161.33 95.61) (end 161.33 96.73) (width 0.25) (layer B.Cu) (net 7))
 (segment (start 161.33 96.73) (end 162.13 97.53) (width 0.25) (layer B.Cu) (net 7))
 (segment (start 162.13 97.53) (end 165.7 97.53) (width 0.25) (layer B.Cu) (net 7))
 (segment (start 166.15 97.08) (end 166.15 95.28) (width 0.25) (layer B.Cu) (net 7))
 (segment (start 165.7 97.53) (end 166.15 97.08) (width 0.25) (layer B.Cu) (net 7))
 (segment (start 166.15 92.39) (end 166.15 92.74) (width 0.25) (layer B.Cu) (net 9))
 (segment (start 163.87 90.11) (end 166.15 92.39) (width 0.25) (layer B.Cu) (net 9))
 (segment (start 149.48 90.11) (end 163.87 90.11) (width 0.25) (layer B.Cu) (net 9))
 (segment (start 148.73 89.36) (end 149.48 90.11) (width 0.25) (layer B.Cu) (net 9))
 (segment (start 148.73 88.01) (end 148.73 89.36) (width 0.25) (layer B.Cu) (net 9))
 (segment (start 158.83 95.61) (end 158.83 96.85) (width 0.25) (layer B.Cu) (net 8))
 (segment (start 159.983999 98.003999) (end 167.836001 98.003999) (width 0.25) (layer B.Cu) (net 8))
 (segment (start 158.83 96.85) (end 159.983999 98.003999) (width 0.25) (layer B.Cu) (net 8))
 (segment (start 167.836001 98.003999) (end 168.75 97.09) (width 0.25) (layer B.Cu) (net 8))
 (segment (start 168.75 97.09) (end 168.75 91.08) (width 0.25) (layer B.Cu) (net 8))
 (segment (start 167.87 90.2) (end 166.15 90.2) (width 0.25) (layer B.Cu) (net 8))
 (segment (start 168.75 91.08) (end 167.87 90.2) (width 0.25) (layer B.Cu) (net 8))
 (segment (start 154.37 84.360002) (end 154.37 83.77) (width 0.25) (layer B.Cu) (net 5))
 (segment (start 145.12 85.12) (end 144.79 84.79) (width 0.25) (layer B.Cu) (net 5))
 (segment (start 153.92 85.12) (end 145.12 85.12) (width 0.25) (layer B.Cu) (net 5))
 (segment (start 154.37 84.67) (end 153.92 85.12) (width 0.25) (layer B.Cu) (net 5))
 (segment (start 144.79 84.79) (end 144.79 82.32) (width 0.25) (layer B.Cu) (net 5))
 (segment (start 154.37 83.77) (end 154.37 84.67) (width 0.25) (layer B.Cu) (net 5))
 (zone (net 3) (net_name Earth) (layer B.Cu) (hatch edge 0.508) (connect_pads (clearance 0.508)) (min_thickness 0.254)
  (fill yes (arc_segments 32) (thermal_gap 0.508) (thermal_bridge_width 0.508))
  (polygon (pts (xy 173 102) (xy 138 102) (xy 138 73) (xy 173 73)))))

